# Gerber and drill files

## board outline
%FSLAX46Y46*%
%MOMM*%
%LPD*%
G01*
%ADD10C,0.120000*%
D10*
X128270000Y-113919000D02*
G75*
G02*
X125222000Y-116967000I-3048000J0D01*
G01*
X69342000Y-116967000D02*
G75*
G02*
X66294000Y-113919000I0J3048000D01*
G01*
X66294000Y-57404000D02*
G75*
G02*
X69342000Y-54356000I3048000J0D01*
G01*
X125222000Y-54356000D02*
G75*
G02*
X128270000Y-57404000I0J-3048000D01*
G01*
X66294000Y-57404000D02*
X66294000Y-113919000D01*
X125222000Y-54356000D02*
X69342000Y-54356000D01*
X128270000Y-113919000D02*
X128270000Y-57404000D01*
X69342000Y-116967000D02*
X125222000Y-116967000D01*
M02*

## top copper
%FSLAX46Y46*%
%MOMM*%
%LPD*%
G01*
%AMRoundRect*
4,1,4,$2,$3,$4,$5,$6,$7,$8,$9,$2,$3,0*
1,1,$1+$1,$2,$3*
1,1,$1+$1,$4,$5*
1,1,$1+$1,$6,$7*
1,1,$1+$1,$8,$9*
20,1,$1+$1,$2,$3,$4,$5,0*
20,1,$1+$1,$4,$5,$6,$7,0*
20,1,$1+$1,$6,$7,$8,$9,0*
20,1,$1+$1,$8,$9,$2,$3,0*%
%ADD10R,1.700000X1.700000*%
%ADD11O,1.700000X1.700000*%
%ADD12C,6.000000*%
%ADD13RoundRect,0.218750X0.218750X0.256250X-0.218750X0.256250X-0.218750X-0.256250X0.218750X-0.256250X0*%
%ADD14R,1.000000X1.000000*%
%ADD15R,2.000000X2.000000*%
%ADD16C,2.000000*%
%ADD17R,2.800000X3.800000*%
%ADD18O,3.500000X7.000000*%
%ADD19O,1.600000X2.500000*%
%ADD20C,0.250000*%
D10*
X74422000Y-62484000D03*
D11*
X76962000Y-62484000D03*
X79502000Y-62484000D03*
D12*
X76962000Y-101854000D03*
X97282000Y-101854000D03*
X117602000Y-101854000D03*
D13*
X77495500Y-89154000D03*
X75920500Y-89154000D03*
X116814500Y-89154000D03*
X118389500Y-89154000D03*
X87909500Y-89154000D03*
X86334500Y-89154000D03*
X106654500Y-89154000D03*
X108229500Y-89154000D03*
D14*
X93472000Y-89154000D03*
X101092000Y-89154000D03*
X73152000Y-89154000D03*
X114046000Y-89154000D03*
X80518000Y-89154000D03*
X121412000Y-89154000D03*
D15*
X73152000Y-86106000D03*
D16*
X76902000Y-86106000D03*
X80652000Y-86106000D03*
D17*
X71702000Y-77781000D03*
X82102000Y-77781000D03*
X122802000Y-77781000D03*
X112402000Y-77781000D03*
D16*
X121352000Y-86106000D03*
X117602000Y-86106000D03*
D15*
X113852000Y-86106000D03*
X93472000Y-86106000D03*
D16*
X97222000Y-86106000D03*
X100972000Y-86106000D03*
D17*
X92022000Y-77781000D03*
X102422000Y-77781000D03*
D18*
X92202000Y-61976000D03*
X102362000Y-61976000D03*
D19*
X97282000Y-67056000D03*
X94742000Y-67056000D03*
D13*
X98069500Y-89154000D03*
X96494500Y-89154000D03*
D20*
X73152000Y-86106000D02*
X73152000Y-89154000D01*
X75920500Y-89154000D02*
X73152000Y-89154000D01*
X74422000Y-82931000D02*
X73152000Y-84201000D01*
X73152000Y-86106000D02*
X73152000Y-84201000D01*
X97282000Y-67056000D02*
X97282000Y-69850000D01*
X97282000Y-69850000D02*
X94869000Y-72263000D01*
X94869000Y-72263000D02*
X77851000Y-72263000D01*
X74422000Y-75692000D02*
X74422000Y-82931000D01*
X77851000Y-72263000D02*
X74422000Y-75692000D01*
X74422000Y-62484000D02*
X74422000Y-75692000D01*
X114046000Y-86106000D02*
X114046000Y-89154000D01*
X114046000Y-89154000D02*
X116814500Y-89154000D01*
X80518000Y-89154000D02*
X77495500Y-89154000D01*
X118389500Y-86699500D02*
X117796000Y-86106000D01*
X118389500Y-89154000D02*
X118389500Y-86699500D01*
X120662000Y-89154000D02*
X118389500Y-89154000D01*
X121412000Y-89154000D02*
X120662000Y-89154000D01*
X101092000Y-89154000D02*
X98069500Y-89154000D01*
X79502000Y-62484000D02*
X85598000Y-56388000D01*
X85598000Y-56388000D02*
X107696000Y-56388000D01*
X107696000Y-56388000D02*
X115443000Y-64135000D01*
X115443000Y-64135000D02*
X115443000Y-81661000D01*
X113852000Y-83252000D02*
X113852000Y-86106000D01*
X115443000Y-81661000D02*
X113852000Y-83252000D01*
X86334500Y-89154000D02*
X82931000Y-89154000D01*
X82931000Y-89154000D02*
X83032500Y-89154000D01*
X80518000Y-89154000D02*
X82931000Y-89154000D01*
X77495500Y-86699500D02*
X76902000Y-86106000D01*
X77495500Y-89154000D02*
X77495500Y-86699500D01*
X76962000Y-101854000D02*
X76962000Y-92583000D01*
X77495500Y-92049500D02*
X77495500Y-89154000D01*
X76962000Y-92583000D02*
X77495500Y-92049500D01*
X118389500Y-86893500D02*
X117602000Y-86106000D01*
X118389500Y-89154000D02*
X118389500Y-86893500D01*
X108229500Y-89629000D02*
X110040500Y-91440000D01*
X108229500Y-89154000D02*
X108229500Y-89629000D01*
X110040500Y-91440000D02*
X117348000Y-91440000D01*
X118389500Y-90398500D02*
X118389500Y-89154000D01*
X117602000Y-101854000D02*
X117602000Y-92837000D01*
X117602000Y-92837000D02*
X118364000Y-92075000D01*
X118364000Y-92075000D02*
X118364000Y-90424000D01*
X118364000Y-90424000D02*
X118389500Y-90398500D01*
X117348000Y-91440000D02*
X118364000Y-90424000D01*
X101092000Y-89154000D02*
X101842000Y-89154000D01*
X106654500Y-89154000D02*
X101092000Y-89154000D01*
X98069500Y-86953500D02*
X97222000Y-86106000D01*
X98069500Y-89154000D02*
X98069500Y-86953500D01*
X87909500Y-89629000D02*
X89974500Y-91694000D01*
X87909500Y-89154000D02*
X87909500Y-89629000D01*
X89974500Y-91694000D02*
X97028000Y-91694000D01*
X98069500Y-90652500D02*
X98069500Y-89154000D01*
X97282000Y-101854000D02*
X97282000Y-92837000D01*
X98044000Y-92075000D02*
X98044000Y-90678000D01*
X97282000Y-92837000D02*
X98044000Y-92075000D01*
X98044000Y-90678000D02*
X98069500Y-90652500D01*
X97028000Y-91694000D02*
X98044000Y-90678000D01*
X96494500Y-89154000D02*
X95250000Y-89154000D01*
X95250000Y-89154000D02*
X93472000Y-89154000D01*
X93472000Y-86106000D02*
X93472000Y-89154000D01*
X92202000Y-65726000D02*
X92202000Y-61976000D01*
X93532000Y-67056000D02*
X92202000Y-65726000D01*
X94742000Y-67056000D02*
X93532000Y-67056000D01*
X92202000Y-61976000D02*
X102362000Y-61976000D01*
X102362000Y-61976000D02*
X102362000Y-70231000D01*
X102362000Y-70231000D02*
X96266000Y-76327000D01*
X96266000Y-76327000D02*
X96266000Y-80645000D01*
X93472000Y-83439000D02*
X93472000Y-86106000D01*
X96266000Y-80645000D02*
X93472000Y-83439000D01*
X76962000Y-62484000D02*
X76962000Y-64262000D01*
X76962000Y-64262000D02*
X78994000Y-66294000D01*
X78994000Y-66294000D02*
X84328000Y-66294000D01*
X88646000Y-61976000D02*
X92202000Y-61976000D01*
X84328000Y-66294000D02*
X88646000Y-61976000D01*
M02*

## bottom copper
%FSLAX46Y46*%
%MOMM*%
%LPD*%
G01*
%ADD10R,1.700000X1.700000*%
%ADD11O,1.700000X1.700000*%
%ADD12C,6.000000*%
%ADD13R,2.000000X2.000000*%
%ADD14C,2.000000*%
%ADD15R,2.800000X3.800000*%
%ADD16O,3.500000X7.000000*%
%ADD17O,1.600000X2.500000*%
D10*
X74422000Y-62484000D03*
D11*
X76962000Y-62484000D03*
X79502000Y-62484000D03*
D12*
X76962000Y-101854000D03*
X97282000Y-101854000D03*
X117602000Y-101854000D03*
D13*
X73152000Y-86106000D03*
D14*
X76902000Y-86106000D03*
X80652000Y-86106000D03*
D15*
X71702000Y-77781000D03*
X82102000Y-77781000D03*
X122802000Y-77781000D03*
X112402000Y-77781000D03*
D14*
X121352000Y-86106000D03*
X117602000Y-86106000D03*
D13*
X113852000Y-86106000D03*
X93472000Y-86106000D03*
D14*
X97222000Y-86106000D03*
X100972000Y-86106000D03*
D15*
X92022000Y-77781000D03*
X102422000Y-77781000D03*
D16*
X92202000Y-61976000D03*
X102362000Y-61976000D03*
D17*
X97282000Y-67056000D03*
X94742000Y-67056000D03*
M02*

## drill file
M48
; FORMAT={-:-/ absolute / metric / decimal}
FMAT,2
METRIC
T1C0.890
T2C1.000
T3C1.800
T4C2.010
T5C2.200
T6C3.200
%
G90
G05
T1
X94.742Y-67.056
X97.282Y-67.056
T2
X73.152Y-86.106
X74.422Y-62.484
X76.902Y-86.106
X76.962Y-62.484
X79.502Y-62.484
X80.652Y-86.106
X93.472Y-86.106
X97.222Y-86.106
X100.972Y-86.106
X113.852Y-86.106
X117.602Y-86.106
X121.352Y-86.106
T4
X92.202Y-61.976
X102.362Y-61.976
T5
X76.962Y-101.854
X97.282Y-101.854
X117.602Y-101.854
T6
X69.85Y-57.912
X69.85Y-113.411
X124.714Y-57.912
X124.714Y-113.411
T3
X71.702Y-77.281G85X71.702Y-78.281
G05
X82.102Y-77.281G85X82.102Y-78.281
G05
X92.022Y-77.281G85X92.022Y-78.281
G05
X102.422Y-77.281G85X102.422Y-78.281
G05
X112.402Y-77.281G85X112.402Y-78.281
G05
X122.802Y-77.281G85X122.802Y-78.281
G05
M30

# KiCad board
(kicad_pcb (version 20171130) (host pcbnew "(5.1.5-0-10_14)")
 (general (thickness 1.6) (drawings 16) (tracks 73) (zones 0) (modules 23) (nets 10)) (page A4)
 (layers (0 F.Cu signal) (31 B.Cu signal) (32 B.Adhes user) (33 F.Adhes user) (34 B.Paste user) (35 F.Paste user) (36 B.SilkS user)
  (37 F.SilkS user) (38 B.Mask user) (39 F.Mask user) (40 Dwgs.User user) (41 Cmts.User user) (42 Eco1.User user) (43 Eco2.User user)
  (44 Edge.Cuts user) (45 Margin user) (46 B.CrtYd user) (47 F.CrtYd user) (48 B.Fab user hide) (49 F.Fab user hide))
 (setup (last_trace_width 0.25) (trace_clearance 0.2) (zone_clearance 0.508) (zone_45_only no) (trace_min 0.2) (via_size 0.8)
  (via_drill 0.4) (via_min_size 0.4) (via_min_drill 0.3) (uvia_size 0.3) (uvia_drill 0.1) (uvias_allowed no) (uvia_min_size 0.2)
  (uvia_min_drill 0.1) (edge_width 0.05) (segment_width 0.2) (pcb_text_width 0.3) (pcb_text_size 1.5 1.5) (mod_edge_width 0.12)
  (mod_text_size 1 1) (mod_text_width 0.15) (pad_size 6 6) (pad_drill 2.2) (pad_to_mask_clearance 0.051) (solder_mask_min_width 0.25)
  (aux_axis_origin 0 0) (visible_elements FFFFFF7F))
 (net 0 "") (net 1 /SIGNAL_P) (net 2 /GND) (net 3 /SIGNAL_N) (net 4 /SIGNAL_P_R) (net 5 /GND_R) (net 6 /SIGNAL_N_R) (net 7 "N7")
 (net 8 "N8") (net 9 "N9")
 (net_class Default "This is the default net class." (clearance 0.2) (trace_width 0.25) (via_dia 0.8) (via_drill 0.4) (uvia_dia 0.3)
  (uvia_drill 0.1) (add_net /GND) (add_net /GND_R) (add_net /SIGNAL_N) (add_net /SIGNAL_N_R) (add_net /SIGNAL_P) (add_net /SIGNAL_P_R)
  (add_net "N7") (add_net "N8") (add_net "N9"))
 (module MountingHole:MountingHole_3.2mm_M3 (layer F.Cu) (at 69.85 57.912)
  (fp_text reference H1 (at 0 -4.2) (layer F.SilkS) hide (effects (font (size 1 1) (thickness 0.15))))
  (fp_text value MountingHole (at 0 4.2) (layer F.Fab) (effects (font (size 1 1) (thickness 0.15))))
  (pad 1 np_thru_hole circle (at 0 0) (size 3.2 3.2) (drill 3.2) (layers *.Cu *.Mask)))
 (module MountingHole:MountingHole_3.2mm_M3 (layer F.Cu) (at 69.85 113.411)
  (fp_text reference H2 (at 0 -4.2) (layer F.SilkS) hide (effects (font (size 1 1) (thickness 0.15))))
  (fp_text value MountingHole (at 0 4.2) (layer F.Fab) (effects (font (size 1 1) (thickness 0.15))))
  (pad 1 np_thru_hole circle (at 0 0) (size 3.2 3.2) (drill 3.2) (layers *.Cu *.Mask)))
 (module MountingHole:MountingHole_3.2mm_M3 (layer F.Cu) (at 124.714 113.411)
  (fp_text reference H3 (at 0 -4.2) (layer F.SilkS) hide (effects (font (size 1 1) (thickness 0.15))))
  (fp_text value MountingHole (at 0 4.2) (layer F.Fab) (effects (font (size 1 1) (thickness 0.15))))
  (pad 1 np_thru_hole circle (at 0 0) (size 3.2 3.2) (drill 3.2) (layers *.Cu *.Mask)))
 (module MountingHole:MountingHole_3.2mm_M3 (layer F.Cu) (at 124.714 57.912)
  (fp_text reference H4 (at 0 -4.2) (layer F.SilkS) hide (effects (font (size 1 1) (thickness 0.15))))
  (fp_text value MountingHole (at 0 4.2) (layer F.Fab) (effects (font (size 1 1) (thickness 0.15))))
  (pad 1 np_thru_hole circle (at 0 0) (size 3.2 3.2) (drill 3.2) (layers *.Cu *.Mask)))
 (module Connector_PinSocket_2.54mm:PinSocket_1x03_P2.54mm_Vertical (layer F.Cu) (at 74.422 62.484 90)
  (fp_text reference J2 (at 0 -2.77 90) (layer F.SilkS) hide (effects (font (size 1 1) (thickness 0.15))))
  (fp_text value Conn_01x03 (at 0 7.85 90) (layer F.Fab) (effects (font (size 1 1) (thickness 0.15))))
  (pad 1 thru_hole rect (at 0 0 90) (size 1.7 1.7) (drill 1) (layers *.Cu *.Mask) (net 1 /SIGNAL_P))
  (pad 2 thru_hole oval (at 0 2.54 90) (size 1.7 1.7) (drill 1) (layers *.Cu *.Mask) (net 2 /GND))
  (pad 3 thru_hole oval (at 0 5.08 90) (size 1.7 1.7) (drill 1) (layers *.Cu *.Mask) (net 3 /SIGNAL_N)))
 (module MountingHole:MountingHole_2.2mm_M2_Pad (layer F.Cu) (at 76.962 101.854)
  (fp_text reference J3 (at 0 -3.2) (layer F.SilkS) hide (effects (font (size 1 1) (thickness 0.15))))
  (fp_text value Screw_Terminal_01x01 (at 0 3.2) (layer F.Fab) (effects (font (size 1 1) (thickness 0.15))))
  (pad 1 thru_hole circle (at 0 0) (size 6 6) (drill 2.2) (layers *.Cu *.Mask) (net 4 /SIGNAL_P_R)))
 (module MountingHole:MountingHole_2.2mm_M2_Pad (layer F.Cu) (at 97.282 101.854)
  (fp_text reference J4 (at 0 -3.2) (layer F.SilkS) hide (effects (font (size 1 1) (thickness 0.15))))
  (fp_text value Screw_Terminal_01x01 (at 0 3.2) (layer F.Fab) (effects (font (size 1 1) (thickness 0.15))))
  (pad 1 thru_hole circle (at 0 0) (size 6 6) (drill 2.2) (layers *.Cu *.Mask) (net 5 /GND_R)))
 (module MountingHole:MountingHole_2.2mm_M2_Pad (layer F.Cu) (at 117.602 101.854)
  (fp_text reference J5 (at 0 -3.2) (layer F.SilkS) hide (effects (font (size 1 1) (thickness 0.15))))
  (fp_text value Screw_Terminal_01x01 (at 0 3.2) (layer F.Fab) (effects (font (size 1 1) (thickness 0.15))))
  (pad 1 thru_hole circle (at 0 0) (size 6 6) (drill 2.2) (layers *.Cu *.Mask) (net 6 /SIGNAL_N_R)))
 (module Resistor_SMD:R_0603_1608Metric (layer F.Cu) (at 76.708 89.154 180)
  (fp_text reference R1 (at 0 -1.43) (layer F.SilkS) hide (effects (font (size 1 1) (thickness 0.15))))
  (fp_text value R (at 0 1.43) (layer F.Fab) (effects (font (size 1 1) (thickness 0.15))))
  (pad 1 smd roundrect (at -0.7875 0 180) (size 0.875 0.95) (layers F.Cu F.Paste F.Mask) (roundrect_rratio 0.25) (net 4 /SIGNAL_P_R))
  (pad 2 smd roundrect (at 0.7875 0 180) (size 0.875 0.95) (layers F.Cu F.Paste F.Mask) (roundrect_rratio 0.25) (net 1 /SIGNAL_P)))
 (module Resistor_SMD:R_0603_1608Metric (layer F.Cu) (at 117.602 89.154 180)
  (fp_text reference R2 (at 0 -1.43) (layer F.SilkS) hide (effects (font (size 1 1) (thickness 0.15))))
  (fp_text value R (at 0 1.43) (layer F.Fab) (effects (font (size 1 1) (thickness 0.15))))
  (pad 2 smd roundrect (at 0.7875 0 180) (size 0.875 0.95) (layers F.Cu F.Paste F.Mask) (roundrect_rratio 0.25) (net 3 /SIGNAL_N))
  (pad 1 smd roundrect (at -0.7875 0 180) (size 0.875 0.95) (layers F.Cu F.Paste F.Mask) (roundrect_rratio 0.25) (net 6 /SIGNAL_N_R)))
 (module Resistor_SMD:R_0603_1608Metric (layer F.Cu) (at 87.122 89.154 180)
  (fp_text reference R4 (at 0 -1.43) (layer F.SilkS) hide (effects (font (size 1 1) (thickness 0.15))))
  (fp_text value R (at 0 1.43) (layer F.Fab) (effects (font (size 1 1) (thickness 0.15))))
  (pad 1 smd roundrect (at -0.7875 0 180) (size 0.875 0.95) (layers F.Cu F.Paste F.Mask) (roundrect_rratio 0.25) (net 5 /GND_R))
  (pad 2 smd roundrect (at 0.7875 0 180) (size 0.875 0.95) (layers F.Cu F.Paste F.Mask) (roundrect_rratio 0.25) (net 4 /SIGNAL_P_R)))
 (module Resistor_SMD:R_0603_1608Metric (layer F.Cu) (at 107.442 89.154 180)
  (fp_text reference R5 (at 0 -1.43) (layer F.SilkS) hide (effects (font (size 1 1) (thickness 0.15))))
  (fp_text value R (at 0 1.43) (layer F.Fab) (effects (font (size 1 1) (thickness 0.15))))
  (pad 2 smd roundrect (at 0.7875 0 180) (size 0.875 0.95) (layers F.Cu F.Paste F.Mask) (roundrect_rratio 0.25) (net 5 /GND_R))
  (pad 1 smd roundrect (at -0.7875 0 180) (size 0.875 0.95) (layers F.Cu F.Paste F.Mask) (roundrect_rratio 0.25) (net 6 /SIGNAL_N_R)))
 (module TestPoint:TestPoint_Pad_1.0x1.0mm (layer F.Cu) (at 93.472 89.154)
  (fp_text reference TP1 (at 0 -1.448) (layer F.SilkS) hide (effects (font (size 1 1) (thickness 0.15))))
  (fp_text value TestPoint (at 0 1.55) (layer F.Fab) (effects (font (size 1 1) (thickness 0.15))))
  (pad 1 smd rect (at 0 0) (size 1 1) (layers F.Cu F.Mask) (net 2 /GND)))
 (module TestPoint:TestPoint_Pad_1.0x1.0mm (layer F.Cu) (at 101.092 89.154)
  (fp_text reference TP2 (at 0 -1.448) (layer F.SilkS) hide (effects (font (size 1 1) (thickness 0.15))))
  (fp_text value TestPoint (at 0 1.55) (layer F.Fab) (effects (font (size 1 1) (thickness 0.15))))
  (pad 1 smd rect (at 0 0) (size 1 1) (layers F.Cu F.Mask) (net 5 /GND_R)))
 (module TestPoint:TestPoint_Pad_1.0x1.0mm (layer F.Cu) (at 73.152 89.154)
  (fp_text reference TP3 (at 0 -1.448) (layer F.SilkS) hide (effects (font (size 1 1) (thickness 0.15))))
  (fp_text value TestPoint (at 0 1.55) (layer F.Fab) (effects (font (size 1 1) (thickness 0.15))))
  (pad 1 smd rect (at 0 0) (size 1 1) (layers F.Cu F.Mask) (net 1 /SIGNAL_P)))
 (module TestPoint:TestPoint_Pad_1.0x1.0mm (layer F.Cu) (at 114.046 89.154)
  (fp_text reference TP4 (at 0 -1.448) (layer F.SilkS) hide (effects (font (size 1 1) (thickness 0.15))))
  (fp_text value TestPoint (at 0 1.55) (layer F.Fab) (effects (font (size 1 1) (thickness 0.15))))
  (pad 1 smd rect (at 0 0) (size 1 1) (layers F.Cu F.Mask) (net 3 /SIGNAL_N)))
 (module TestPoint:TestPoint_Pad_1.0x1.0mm (layer F.Cu) (at 80.518 89.154)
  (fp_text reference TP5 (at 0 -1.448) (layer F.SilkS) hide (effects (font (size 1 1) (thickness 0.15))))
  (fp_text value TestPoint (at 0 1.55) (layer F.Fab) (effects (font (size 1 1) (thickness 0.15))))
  (pad 1 smd rect (at 0 0) (size 1 1) (layers F.Cu F.Mask) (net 4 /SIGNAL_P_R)))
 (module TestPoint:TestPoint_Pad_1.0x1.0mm (layer F.Cu) (at 121.412 89.154)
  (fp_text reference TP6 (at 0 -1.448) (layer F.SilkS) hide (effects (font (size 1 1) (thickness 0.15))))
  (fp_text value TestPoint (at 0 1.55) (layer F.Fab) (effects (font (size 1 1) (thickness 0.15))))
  (pad 1 smd rect (at 0 0) (size 1 1) (layers F.Cu F.Mask) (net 6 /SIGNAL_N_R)))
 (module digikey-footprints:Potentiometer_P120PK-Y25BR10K (layer F.Cu) (at 73.152 86.106)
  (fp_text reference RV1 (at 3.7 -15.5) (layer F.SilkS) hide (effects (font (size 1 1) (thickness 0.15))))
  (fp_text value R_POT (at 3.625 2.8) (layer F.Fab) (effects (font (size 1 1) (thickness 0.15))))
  (pad 1 thru_hole rect (at 0 0) (size 2 2) (drill 1) (layers *.Cu *.Mask) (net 1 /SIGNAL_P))
  (pad 2 thru_hole circle (at 3.75 0) (size 2 2) (drill 1) (layers *.Cu *.Mask) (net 4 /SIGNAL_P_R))
  (pad 3 thru_hole circle (at 7.5 0) (size 2 2) (drill 1) (layers *.Cu *.Mask) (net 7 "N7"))
  (pad 4 thru_hole rect (at -1.45 -8.325) (size 2.8 3.8) (drill oval 1.8 2.8) (layers *.Cu *.Mask))
  (pad 4 thru_hole rect (at 8.95 -8.325) (size 2.8 3.8) (drill oval 1.8 2.8) (layers *.Cu *.Mask)))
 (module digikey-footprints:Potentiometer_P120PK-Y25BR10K (layer F.Cu) (at 113.852 86.106)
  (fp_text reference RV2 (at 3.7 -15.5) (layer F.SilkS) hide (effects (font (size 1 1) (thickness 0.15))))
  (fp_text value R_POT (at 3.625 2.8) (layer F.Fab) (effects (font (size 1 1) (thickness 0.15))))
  (pad 4 thru_hole rect (at 8.95 -8.325) (size 2.8 3.8) (drill oval 1.8 2.8) (layers *.Cu *.Mask))
  (pad 4 thru_hole rect (at -1.45 -8.325) (size 2.8 3.8) (drill oval 1.8 2.8) (layers *.Cu *.Mask))
  (pad 3 thru_hole circle (at 7.5 0) (size 2 2) (drill 1) (layers *.Cu *.Mask) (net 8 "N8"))
  (pad 2 thru_hole circle (at 3.75 0) (size 2 2) (drill 1) (layers *.Cu *.Mask) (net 6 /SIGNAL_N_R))
  (pad 1 thru_hole rect (at 0 0) (size 2 2) (drill 1) (layers *.Cu *.Mask) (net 3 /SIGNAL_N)))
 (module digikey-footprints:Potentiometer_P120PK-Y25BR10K (layer F.Cu) (at 93.472 86.106)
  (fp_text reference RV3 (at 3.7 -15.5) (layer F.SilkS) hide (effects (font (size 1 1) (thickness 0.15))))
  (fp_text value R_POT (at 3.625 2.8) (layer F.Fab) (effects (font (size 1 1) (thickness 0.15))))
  (pad 1 thru_hole rect (at 0 0) (size 2 2) (drill 1) (layers *.Cu *.Mask) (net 2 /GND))
  (pad 2 thru_hole circle (at 3.75 0) (size 2 2) (drill 1) (layers *.Cu *.Mask) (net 5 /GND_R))
  (pad 3 thru_hole circle (at 7.5 0) (size 2 2) (drill 1) (layers *.Cu *.Mask) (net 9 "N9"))
  (pad 4 thru_hole rect (at -1.45 -8.325) (size 2.8 3.8) (drill oval 1.8 2.8) (layers *.Cu *.Mask))
  (pad 4 thru_hole rect (at 8.95 -8.325) (size 2.8 3.8) (drill oval 1.8 2.8) (layers *.Cu *.Mask)))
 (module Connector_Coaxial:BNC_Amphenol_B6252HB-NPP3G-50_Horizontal (layer F.Cu) (at 97.282 67.056)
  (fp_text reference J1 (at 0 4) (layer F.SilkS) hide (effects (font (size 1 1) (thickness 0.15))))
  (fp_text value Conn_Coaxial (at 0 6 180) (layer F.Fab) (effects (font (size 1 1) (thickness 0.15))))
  (pad 2 thru_hole oval (at -5.08 -5.08) (size 3.5 7) (drill 2.01) (layers *.Cu *.Mask) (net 2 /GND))
  (pad 2 thru_hole oval (at 5.08 -5.08) (size 3.5 7) (drill 2.01) (layers *.Cu *.Mask) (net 2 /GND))
  (pad 1 thru_hole oval (at 0 0) (size 1.6 2.5) (drill 0.89) (layers *.Cu *.Mask) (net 1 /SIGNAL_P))
  (pad 2 thru_hole oval (at -2.54 0) (size 1.6 2.5) (drill 0.89) (layers *.Cu *.Mask) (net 2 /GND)))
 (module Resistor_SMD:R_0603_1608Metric (layer F.Cu) (at 97.282 89.154 180)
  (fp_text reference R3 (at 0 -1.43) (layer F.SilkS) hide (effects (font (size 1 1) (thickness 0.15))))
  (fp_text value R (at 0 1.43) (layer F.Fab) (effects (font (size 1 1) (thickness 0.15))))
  (pad 1 smd roundrect (at -0.7875 0 180) (size 0.875 0.95) (layers F.Cu F.Paste F.Mask) (roundrect_rratio 0.25) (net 5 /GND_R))
  (pad 2 smd roundrect (at 0.7875 0 180) (size 0.875 0.95) (layers F.Cu F.Paste F.Mask) (roundrect_rratio 0.25) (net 2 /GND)))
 (gr_arc (start 125.222 113.919) (end 125.222 116.967) (angle -90) (layer Edge.Cuts) (width 0.12))
 (gr_arc (start 69.342 113.919) (end 66.294 113.919) (angle -90) (layer Edge.Cuts) (width 0.12))
 (gr_arc (start 69.342 57.404) (end 69.342 54.356) (angle -90) (layer Edge.Cuts) (width 0.12))
 (gr_arc (start 125.222 57.404) (end 128.27 57.404) (angle -90) (layer Edge.Cuts) (width 0.12))
 (gr_line (start 66.294 57.404) (end 66.294 113.919) (layer Edge.Cuts) (width 0.12))
 (gr_line (start 125.222 54.356) (end 69.342 54.356) (layer Edge.Cuts) (width 0.12))
 (gr_line (start 128.27 113.919) (end 128.27 57.404) (layer Edge.Cuts) (width 0.12))
 (gr_line (start 69.342 116.967) (end 125.222 116.967) (layer Edge.Cuts) (width 0.12))
 (segment (start 73.152 86.106) (end 73.152 89.154) (width 0.25) (layer F.Cu) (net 1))
 (segment (start 75.9205 89.154) (end 73.152 89.154) (width 0.25) (layer F.Cu) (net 1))
 (segment (start 74.422 82.931) (end 73.152 84.201) (width 0.25) (layer F.Cu) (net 1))
 (segment (start 73.152 86.106) (end 73.152 84.201) (width 0.25) (layer F.Cu) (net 1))
 (segment (start 97.282 67.056) (end 97.282 69.85) (width 0.25) (layer F.Cu) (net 1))
 (segment (start 97.282 69.85) (end 94.869 72.263) (width 0.25) (layer F.Cu) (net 1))
 (segment (start 94.869 72.263) (end 77.851 72.263) (width 0.25) (layer F.Cu) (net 1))
 (segment (start 74.422 75.692) (end 74.422 82.931) (width 0.25) (layer F.Cu) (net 1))
 (segment (start 77.851 72.263) (end 74.422 75.692) (width 0.25) (layer F.Cu) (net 1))
 (segment (start 74.422 62.484) (end 74.422 75.692) (width 0.25) (layer F.Cu) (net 1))
 (segment (start 114.046 86.106) (end 114.046 89.154) (width 0.25) (layer F.Cu) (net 3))
 (segment (start 114.046 89.154) (end 116.8145 89.154) (width 0.25) (layer F.Cu) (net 3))
 (segment (start 80.518 89.154) (end 77.4955 89.154) (width 0.25) (layer F.Cu) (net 4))
 (segment (start 118.3895 86.6995) (end 117.796 86.106) (width 0.25) (layer F.Cu) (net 6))
 (segment (start 118.3895 89.154) (end 118.3895 86.6995) (width 0.25) (layer F.Cu) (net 6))
 (segment (start 120.662 89.154) (end 118.3895 89.154) (width 0.25) (layer F.Cu) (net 6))
 (segment (start 121.412 89.154) (end 120.662 89.154) (width 0.25) (layer F.Cu) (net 6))
 (segment (start 101.092 89.154) (end 98.0695 89.154) (width 0.25) (layer F.Cu) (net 5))
 (segment (start 79.502 62.484) (end 85.598 56.388) (width 0.25) (layer F.Cu) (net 3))
 (segment (start 85.598 56.388) (end 107.696 56.388) (width 0.25) (layer F.Cu) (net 3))
 (segment (start 107.696 56.388) (end 115.443 64.135) (width 0.25) (layer F.Cu) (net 3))
 (segment (start 115.443 64.135) (end 115.443 81.661) (width 0.25) (layer F.Cu) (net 3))
 (segment (start 113.852 83.252) (end 113.852 86.106) (width 0.25) (layer F.Cu) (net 3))
 (segment (start 115.443 81.661) (end 113.852 83.252) (width 0.25) (layer F.Cu) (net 3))
 (segment (start 86.3345 89.154) (end 82.931 89.154) (width 0.25) (layer F.Cu) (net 4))
 (segment (start 82.931 89.154) (end 83.0325 89.154) (width 0.25) (layer F.Cu) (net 4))
 (segment (start 80.518 89.154) (end 82.931 89.154) (width 0.25) (layer F.Cu) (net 4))
 (segment (start 77.4955 86.6995) (end 76.902 86.106) (width 0.25) (layer F.Cu) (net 4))
 (segment (start 77.4955 89.154) (end 77.4955 86.6995) (width 0.25) (layer F.Cu) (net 4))
 (segment (start 76.962 101.854) (end 76.962 92.583) (width 0.25) (layer F.Cu) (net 4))
 (segment (start 77.4955 92.0495) (end 77.4955 89.154) (width 0.25) (layer F.Cu) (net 4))
 (segment (start 76.962 92.583) (end 77.4955 92.0495) (width 0.25) (layer F.Cu) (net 4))
 (segment (start 118.3895 86.8935) (end 117.602 86.106) (width 0.25) (layer F.Cu) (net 6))
 (segment (start 118.3895 89.154) (end 118.3895 86.8935) (width 0.25) (layer F.Cu) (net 6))
 (segment (start 108.2295 89.629) (end 110.0405 91.44) (width 0.25) (layer F.Cu) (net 6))
 (segment (start 108.2295 89.154) (end 108.2295 89.629) (width 0.25) (layer F.Cu) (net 6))
 (segment (start 110.0405 91.44) (end 117.348 91.44) (width 0.25) (layer F.Cu) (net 6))
 (segment (start 118.3895 90.3985) (end 118.3895 89.154) (width 0.25) (layer F.Cu) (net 6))
 (segment (start 117.602 101.854) (end 117.602 92.837) (width 0.25) (layer F.Cu) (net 6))
 (segment (start 117.602 92.837) (end 118.364 92.075) (width 0.25) (layer F.Cu) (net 6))
 (segment (start 118.364 92.075) (end 118.364 90.424) (width 0.25) (layer F.Cu) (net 6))
 (segment (start 118.364 90.424) (end 118.3895 90.3985) (width 0.25) (layer F.Cu) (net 6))
 (segment (start 117.348 91.44) (end 118.364 90.424) (width 0.25) (layer F.Cu) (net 6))
 (segment (start 101.092 89.154) (end 101.842 89.154) (width 0.25) (layer F.Cu) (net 5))
 (segment (start 106.6545 89.154) (end 101.092 89.154) (width 0.25) (layer F.Cu) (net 5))
 (segment (start 98.0695 86.9535) (end 97.222 86.106) (width 0.25) (layer F.Cu) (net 5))
 (segment (start 98.0695 89.154) (end 98.0695 86.9535) (width 0.25) (layer F.Cu) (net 5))
 (segment (start 87.9095 89.629) (end 89.9745 91.694) (width 0.25) (layer F.Cu) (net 5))
 (segment (start 87.9095 89.154) (end 87.9095 89.629) (width 0.25) (layer F.Cu) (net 5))
 (segment (start 89.9745 91.694) (end 97.028 91.694) (width 0.25) (layer F.Cu) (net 5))
 (segment (start 98.0695 90.6525) (end 98.0695 89.154) (width 0.25) (layer F.Cu) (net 5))
 (segment (start 97.282 101.854) (end 97.282 92.837) (width 0.25) (layer F.Cu) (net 5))
 (segment (start 98.044 92.075) (end 98.044 90.678) (width 0.25) (layer F.Cu) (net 5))
 (segment (start 97.282 92.837) (end 98.044 92.075) (width 0.25) (layer F.Cu) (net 5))
 (segment (start 98.044 90.678) (end 98.0695 90.6525) (width 0.25) (layer F.Cu) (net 5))
 (segment (start 97.028 91.694) (end 98.044 90.678) (width 0.25) (layer F.Cu) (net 5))
 (segment (start 96.4945 89.154) (end 95.25 89.154) (width 0.25) (layer F.Cu) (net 2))
 (segment (start 95.25 89.154) (end 93.472 89.154) (width 0.25) (layer F.Cu) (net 2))
 (segment (start 93.472 86.106) (end 93.472 89.154) (width 0.25) (layer F.Cu) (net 2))
 (segment (start 92.202 65.726) (end 92.202 61.976) (width 0.25) (layer F.Cu) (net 2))
 (segment (start 93.532 67.056) (end 92.202 65.726) (width 0.25) (layer F.Cu) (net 2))
 (segment (start 94.742 67.056) (end 93.532 67.056) (width 0.25) (layer F.Cu) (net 2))
 (segment (start 92.202 61.976) (end 102.362 61.976) (width 0.25) (layer F.Cu) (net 2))
 (segment (start 102.362 61.976) (end 102.362 70.231) (width 0.25) (layer F.Cu) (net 2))
 (segment (start 102.362 70.231) (end 96.266 76.327) (width 0.25) (layer F.Cu) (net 2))
 (segment (start 96.266 76.327) (end 96.266 80.645) (width 0.25) (layer F.Cu) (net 2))
 (segment (start 93.472 83.439) (end 93.472 86.106) (width 0.25) (layer F.Cu) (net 2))
 (segment (start 96.266 80.645) (end 93.472 83.439) (width 0.25) (layer F.Cu) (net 2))
 (segment (start 76.962 62.484) (end 76.962 64.262) (width 0.25) (layer F.Cu) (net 2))
 (segment (start 76.962 64.262) (end 78.994 66.294) (width 0.25) (layer F.Cu) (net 2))
 (segment (start 78.994 66.294) (end 84.328 66.294) (width 0.25) (layer F.Cu) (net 2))
 (segment (start 88.646 61.976) (end 92.202 61.976) (width 0.25) (layer F.Cu) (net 2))
 (segment (start 84.328 66.294) (end 88.646 61.976) (width 0.25) (layer F.Cu) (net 2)))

